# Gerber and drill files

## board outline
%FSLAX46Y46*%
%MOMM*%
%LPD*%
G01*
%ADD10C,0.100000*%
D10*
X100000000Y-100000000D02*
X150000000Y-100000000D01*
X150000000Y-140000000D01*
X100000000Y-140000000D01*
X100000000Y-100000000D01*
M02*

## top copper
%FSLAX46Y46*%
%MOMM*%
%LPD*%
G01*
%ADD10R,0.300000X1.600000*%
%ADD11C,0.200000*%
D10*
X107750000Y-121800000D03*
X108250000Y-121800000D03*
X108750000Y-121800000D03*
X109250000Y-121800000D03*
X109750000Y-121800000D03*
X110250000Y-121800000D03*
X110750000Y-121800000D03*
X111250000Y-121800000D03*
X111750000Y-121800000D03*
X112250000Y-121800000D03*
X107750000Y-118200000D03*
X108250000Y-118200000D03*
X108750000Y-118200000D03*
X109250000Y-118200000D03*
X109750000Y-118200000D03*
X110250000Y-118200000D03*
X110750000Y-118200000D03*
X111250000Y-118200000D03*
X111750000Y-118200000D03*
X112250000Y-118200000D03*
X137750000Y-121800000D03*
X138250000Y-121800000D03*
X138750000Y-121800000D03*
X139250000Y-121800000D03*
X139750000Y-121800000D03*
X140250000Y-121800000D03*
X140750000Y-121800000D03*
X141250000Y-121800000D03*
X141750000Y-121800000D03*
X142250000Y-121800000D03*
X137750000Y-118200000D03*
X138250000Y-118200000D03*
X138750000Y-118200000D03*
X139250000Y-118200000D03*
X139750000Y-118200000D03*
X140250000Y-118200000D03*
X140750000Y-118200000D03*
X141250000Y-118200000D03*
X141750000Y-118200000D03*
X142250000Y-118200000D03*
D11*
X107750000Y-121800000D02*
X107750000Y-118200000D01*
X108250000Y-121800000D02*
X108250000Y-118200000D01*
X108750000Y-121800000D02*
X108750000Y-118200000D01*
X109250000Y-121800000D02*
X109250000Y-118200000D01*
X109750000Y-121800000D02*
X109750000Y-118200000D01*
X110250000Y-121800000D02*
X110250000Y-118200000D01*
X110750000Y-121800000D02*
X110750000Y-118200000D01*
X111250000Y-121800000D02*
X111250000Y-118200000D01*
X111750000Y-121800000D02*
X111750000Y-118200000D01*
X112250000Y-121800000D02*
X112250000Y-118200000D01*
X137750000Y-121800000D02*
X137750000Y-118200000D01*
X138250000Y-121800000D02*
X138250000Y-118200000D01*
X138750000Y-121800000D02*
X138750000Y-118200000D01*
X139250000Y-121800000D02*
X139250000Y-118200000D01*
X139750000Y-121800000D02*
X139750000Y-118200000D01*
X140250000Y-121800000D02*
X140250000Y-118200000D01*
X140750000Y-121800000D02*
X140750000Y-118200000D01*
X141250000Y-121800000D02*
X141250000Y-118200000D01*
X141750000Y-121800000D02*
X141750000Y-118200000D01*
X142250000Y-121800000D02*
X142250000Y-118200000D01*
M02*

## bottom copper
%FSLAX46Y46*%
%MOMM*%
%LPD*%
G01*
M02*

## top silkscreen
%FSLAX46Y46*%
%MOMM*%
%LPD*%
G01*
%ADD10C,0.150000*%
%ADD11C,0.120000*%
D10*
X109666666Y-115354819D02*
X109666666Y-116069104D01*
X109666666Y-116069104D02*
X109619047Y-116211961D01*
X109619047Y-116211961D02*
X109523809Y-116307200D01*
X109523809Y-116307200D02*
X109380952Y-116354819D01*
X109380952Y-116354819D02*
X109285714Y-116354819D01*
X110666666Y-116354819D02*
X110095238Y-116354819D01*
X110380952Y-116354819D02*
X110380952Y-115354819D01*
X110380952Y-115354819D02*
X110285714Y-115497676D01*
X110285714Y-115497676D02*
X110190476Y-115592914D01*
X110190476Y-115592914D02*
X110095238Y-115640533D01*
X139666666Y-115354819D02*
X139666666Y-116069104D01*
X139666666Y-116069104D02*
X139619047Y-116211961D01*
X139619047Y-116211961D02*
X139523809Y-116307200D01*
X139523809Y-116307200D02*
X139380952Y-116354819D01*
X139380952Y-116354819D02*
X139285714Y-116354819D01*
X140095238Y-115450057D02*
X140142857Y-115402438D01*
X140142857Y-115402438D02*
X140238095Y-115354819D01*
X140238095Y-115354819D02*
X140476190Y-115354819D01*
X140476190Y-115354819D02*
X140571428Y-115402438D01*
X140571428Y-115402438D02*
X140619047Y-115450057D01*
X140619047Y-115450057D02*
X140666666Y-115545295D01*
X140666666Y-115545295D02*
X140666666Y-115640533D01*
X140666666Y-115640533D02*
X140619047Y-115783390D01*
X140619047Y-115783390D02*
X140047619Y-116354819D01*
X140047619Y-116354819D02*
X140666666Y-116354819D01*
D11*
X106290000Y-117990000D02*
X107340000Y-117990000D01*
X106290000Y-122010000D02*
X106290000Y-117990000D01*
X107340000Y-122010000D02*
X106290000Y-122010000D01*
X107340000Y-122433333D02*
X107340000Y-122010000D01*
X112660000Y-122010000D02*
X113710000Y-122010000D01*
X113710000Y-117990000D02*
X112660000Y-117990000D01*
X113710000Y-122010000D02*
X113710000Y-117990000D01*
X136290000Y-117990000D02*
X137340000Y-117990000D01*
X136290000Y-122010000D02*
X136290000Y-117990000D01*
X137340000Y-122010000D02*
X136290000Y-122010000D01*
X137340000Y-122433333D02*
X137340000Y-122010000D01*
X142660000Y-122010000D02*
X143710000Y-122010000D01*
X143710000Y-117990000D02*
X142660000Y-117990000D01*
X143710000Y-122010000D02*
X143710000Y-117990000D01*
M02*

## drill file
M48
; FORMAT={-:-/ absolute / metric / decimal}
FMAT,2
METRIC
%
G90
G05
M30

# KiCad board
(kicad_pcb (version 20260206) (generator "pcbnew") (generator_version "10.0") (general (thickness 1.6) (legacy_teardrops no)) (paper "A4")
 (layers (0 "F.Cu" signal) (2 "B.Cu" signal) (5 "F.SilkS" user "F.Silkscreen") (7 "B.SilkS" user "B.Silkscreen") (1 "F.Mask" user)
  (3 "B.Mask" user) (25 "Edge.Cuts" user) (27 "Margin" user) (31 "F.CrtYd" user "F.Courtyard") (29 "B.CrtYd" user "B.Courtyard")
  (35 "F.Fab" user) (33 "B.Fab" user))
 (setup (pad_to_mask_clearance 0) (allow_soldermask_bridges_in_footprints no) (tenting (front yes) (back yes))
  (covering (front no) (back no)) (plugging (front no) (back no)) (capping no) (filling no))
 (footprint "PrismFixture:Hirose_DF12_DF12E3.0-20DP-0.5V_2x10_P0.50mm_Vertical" (layer "F.Cu") (at 110 120)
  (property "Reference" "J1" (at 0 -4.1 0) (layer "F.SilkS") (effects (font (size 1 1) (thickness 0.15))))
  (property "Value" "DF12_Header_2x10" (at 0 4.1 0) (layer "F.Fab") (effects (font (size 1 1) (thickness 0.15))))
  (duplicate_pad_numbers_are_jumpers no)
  (fp_line (start -3.71 -2.01) (end -2.66 -2.01) (stroke (width 0.12) (type solid)) (layer "F.SilkS"))
  (fp_line (start -3.71 2.01) (end -3.71 -2.01) (stroke (width 0.12) (type solid)) (layer "F.SilkS"))
  (fp_line (start -2.66 2.01) (end -3.71 2.01) (stroke (width 0.12) (type solid)) (layer "F.SilkS"))
  (fp_line (start -2.66 2.433333) (end -2.66 2.01) (stroke (width 0.12) (type solid)) (layer "F.SilkS"))
  (fp_line (start 2.66 2.01) (end 3.71 2.01) (stroke (width 0.12) (type solid)) (layer "F.SilkS"))
  (fp_line (start 3.71 -2.01) (end 2.66 -2.01) (stroke (width 0.12) (type solid)) (layer "F.SilkS"))
  (fp_line (start 3.71 2.01) (end 3.71 -2.01) (stroke (width 0.12) (type solid)) (layer "F.SilkS"))
  (pad "" smd rect (at -2.25 -2) (size 0.28 1.2) (layers "F.Paste"))
  (pad "" smd rect (at -2.25 2) (size 0.28 1.2) (layers "F.Paste"))
  (pad "" smd rect (at -1.75 -2) (size 0.28 1.2) (layers "F.Paste"))
  (pad "" smd rect (at -1.75 2) (size 0.28 1.2) (layers "F.Paste"))
  (pad "" smd rect (at -1.25 -2) (size 0.28 1.2) (layers "F.Paste"))
  (pad "" smd rect (at -1.25 2) (size 0.28 1.2) (layers "F.Paste"))
  (pad "" smd rect (at -0.75 -2) (size 0.28 1.2) (layers "F.Paste"))
  (pad "" smd rect (at -0.75 2) (size 0.28 1.2) (layers "F.Paste"))
  (pad "" smd rect (at -0.25 -2) (size 0.28 1.2) (layers "F.Paste"))
  (pad "" smd rect (at -0.25 2) (size 0.28 1.2) (layers "F.Paste"))
  (pad "" smd rect (at 0.25 -2) (size 0.28 1.2) (layers "F.Paste"))
  (pad "" smd rect (at 0.25 2) (size 0.28 1.2) (layers "F.Paste"))
  (pad "" smd rect (at 0.75 -2) (size 0.28 1.2) (layers "F.Paste"))
  (pad "" smd rect (at 0.75 2) (size 0.28 1.2) (layers "F.Paste"))
  (pad "" smd rect (at 1.25 -2) (size 0.28 1.2) (layers "F.Paste"))
  (pad "" smd rect (at 1.25 2) (size 0.28 1.2) (layers "F.Paste"))
  (pad "" smd rect (at 1.75 -2) (size 0.28 1.2) (layers "F.Paste"))
  (pad "" smd rect (at 1.75 2) (size 0.28 1.2) (layers "F.Paste"))
  (pad "" smd rect (at 2.25 -2) (size 0.28 1.2) (layers "F.Paste"))
  (pad "" smd rect (at 2.25 2) (size 0.28 1.2) (layers "F.Paste"))
  (pad "1" smd rect (at -2.25 1.8) (size 0.3 1.6) (layers "F.Cu" "F.Mask") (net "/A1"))
  (pad "2" smd rect (at -1.75 1.8) (size 0.3 1.6) (layers "F.Cu" "F.Mask") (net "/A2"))
  (pad "3" smd rect (at -1.25 1.8) (size 0.3 1.6) (layers "F.Cu" "F.Mask") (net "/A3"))
  (pad "4" smd rect (at -0.75 1.8) (size 0.3 1.6) (layers "F.Cu" "F.Mask") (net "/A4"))
  (pad "5" smd rect (at -0.25 1.8) (size 0.3 1.6) (layers "F.Cu" "F.Mask") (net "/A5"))
  (pad "6" smd rect (at 0.25 1.8) (size 0.3 1.6) (layers "F.Cu" "F.Mask") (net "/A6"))
  (pad "7" smd rect (at 0.75 1.8) (size 0.3 1.6) (layers "F.Cu" "F.Mask") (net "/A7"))
  (pad "8" smd rect (at 1.25 1.8) (size 0.3 1.6) (layers "F.Cu" "F.Mask") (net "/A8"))
  (pad "9" smd rect (at 1.75 1.8) (size 0.3 1.6) (layers "F.Cu" "F.Mask") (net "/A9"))
  (pad "10" smd rect (at 2.25 1.8) (size 0.3 1.6) (layers "F.Cu" "F.Mask") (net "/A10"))
  (pad "11" smd rect (at -2.25 -1.8) (size 0.3 1.6) (layers "F.Cu" "F.Mask") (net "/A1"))
  (pad "12" smd rect (at -1.75 -1.8) (size 0.3 1.6) (layers "F.Cu" "F.Mask") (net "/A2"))
  (pad "13" smd rect (at -1.25 -1.8) (size 0.3 1.6) (layers "F.Cu" "F.Mask") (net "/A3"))
  (pad "14" smd rect (at -0.75 -1.8) (size 0.3 1.6) (layers "F.Cu" "F.Mask") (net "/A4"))
  (pad "15" smd rect (at -0.25 -1.8) (size 0.3 1.6) (layers "F.Cu" "F.Mask") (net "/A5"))
  (pad "16" smd rect (at 0.25 -1.8) (size 0.3 1.6) (layers "F.Cu" "F.Mask") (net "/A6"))
  (pad "17" smd rect (at 0.75 -1.8) (size 0.3 1.6) (layers "F.Cu" "F.Mask") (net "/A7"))
  (pad "18" smd rect (at 1.25 -1.8) (size 0.3 1.6) (layers "F.Cu" "F.Mask") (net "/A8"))
  (pad "19" smd rect (at 1.75 -1.8) (size 0.3 1.6) (layers "F.Cu" "F.Mask") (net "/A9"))
  (pad "20" smd rect (at 2.25 -1.8) (size 0.3 1.6) (layers "F.Cu" "F.Mask") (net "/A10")))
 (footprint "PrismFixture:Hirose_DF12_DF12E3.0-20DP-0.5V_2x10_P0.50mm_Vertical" (layer "F.Cu") (at 140 120)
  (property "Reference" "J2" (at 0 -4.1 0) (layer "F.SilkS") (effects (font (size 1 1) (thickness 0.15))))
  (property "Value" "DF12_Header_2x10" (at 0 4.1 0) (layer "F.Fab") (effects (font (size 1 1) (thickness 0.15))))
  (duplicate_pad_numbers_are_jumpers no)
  (fp_line (start -3.71 -2.01) (end -2.66 -2.01) (stroke (width 0.12) (type solid)) (layer "F.SilkS"))
  (fp_line (start -3.71 2.01) (end -3.71 -2.01) (stroke (width 0.12) (type solid)) (layer "F.SilkS"))
  (fp_line (start -2.66 2.01) (end -3.71 2.01) (stroke (width 0.12) (type solid)) (layer "F.SilkS"))
  (fp_line (start -2.66 2.433333) (end -2.66 2.01) (stroke (width 0.12) (type solid)) (layer "F.SilkS"))
  (fp_line (start 2.66 2.01) (end 3.71 2.01) (stroke (width 0.12) (type solid)) (layer "F.SilkS"))
  (fp_line (start 3.71 -2.01) (end 2.66 -2.01) (stroke (width 0.12) (type solid)) (layer "F.SilkS"))
  (fp_line (start 3.71 2.01) (end 3.71 -2.01) (stroke (width 0.12) (type solid)) (layer "F.SilkS"))
  (pad "" smd rect (at -2.25 -2) (size 0.28 1.2) (layers "F.Paste"))
  (pad "" smd rect (at -2.25 2) (size 0.28 1.2) (layers "F.Paste"))
  (pad "" smd rect (at -1.75 -2) (size 0.28 1.2) (layers "F.Paste"))
  (pad "" smd rect (at -1.75 2) (size 0.28 1.2) (layers "F.Paste"))
  (pad "" smd rect (at -1.25 -2) (size 0.28 1.2) (layers "F.Paste"))
  (pad "" smd rect (at -1.25 2) (size 0.28 1.2) (layers "F.Paste"))
  (pad "" smd rect (at -0.75 -2) (size 0.28 1.2) (layers "F.Paste"))
  (pad "" smd rect (at -0.75 2) (size 0.28 1.2) (layers "F.Paste"))
  (pad "" smd rect (at -0.25 -2) (size 0.28 1.2) (layers "F.Paste"))
  (pad "" smd rect (at -0.25 2) (size 0.28 1.2) (layers "F.Paste"))
  (pad "" smd rect (at 0.25 -2) (size 0.28 1.2) (layers "F.Paste"))
  (pad "" smd rect (at 0.25 2) (size 0.28 1.2) (layers "F.Paste"))
  (pad "" smd rect (at 0.75 -2) (size 0.28 1.2) (layers "F.Paste"))
  (pad "" smd rect (at 0.75 2) (size 0.28 1.2) (layers "F.Paste"))
  (pad "" smd rect (at 1.25 -2) (size 0.28 1.2) (layers "F.Paste"))
  (pad "" smd rect (at 1.25 2) (size 0.28 1.2) (layers "F.Paste"))
  (pad "" smd rect (at 1.75 -2) (size 0.28 1.2) (layers "F.Paste"))
  (pad "" smd rect (at 1.75 2) (size 0.28 1.2) (layers "F.Paste"))
  (pad "" smd rect (at 2.25 -2) (size 0.28 1.2) (layers "F.Paste"))
  (pad "" smd rect (at 2.25 2) (size 0.28 1.2) (layers "F.Paste"))
  (pad "1" smd rect (at -2.25 1.8) (size 0.3 1.6) (layers "F.Cu" "F.Mask") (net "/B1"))
  (pad "2" smd rect (at -1.75 1.8) (size 0.3 1.6) (layers "F.Cu" "F.Mask") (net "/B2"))
  (pad "3" smd rect (at -1.25 1.8) (size 0.3 1.6) (layers "F.Cu" "F.Mask") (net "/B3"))
  (pad "4" smd rect (at -0.75 1.8) (size 0.3 1.6) (layers "F.Cu" "F.Mask") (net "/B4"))
  (pad "5" smd rect (at -0.25 1.8) (size 0.3 1.6) (layers "F.Cu" "F.Mask") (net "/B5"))
  (pad "6" smd rect (at 0.25 1.8) (size 0.3 1.6) (layers "F.Cu" "F.Mask") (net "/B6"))
  (pad "7" smd rect (at 0.75 1.8) (size 0.3 1.6) (layers "F.Cu" "F.Mask") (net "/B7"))
  (pad "8" smd rect (at 1.25 1.8) (size 0.3 1.6) (layers "F.Cu" "F.Mask") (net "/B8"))
  (pad "9" smd rect (at 1.75 1.8) (size 0.3 1.6) (layers "F.Cu" "F.Mask") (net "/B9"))
  (pad "10" smd rect (at 2.25 1.8) (size 0.3 1.6) (layers "F.Cu" "F.Mask") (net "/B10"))
  (pad "11" smd rect (at -2.25 -1.8) (size 0.3 1.6) (layers "F.Cu" "F.Mask") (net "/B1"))
  (pad "12" smd rect (at -1.75 -1.8) (size 0.3 1.6) (layers "F.Cu" "F.Mask") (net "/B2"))
  (pad "13" smd rect (at -1.25 -1.8) (size 0.3 1.6) (layers "F.Cu" "F.Mask") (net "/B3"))
  (pad "14" smd rect (at -0.75 -1.8) (size 0.3 1.6) (layers "F.Cu" "F.Mask") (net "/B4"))
  (pad "15" smd rect (at -0.25 -1.8) (size 0.3 1.6) (layers "F.Cu" "F.Mask") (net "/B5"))
  (pad "16" smd rect (at 0.25 -1.8) (size 0.3 1.6) (layers "F.Cu" "F.Mask") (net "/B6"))
  (pad "17" smd rect (at 0.75 -1.8) (size 0.3 1.6) (layers "F.Cu" "F.Mask") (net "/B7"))
  (pad "18" smd rect (at 1.25 -1.8) (size 0.3 1.6) (layers "F.Cu" "F.Mask") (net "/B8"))
  (pad "19" smd rect (at 1.75 -1.8) (size 0.3 1.6) (layers "F.Cu" "F.Mask") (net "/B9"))
  (pad "20" smd rect (at 2.25 -1.8) (size 0.3 1.6) (layers "F.Cu" "F.Mask") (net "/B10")))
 (gr_rect (start 100 100) (end 150 140) (stroke (width 0.1) (type solid)) (fill no) (layer "Edge.Cuts"))
 (segment (start 107.75 121.8) (end 107.75 118.2) (width 0.2) (layer "F.Cu") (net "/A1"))
 (segment (start 108.25 121.8) (end 108.25 118.2) (width 0.2) (layer "F.Cu") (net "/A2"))
 (segment (start 108.75 121.8) (end 108.75 118.2) (width 0.2) (layer "F.Cu") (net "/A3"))
 (segment (start 109.25 121.8) (end 109.25 118.2) (width 0.2) (layer "F.Cu") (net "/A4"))
 (segment (start 109.75 121.8) (end 109.75 118.2) (width 0.2) (layer "F.Cu") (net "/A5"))
 (segment (start 110.25 121.8) (end 110.25 118.2) (width 0.2) (layer "F.Cu") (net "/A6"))
 (segment (start 110.75 121.8) (end 110.75 118.2) (width 0.2) (layer "F.Cu") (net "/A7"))
 (segment (start 111.25 121.8) (end 111.25 118.2) (width 0.2) (layer "F.Cu") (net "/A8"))
 (segment (start 111.75 121.8) (end 111.75 118.2) (width 0.2) (layer "F.Cu") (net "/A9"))
 (segment (start 112.25 121.8) (end 112.25 118.2) (width 0.2) (layer "F.Cu") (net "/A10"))
 (segment (start 137.75 121.8) (end 137.75 118.2) (width 0.2) (layer "F.Cu") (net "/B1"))
 (segment (start 138.25 121.8) (end 138.25 118.2) (width 0.2) (layer "F.Cu") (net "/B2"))
 (segment (start 138.75 121.8) (end 138.75 118.2) (width 0.2) (layer "F.Cu") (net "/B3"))
 (segment (start 139.25 121.8) (end 139.25 118.2) (width 0.2) (layer "F.Cu") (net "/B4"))
 (segment (start 139.75 121.8) (end 139.75 118.2) (width 0.2) (layer "F.Cu") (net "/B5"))
 (segment (start 140.25 121.8) (end 140.25 118.2) (width 0.2) (layer "F.Cu") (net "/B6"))
 (segment (start 140.75 121.8) (end 140.75 118.2) (width 0.2) (layer "F.Cu") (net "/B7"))
 (segment (start 141.25 121.8) (end 141.25 118.2) (width 0.2) (layer "F.Cu") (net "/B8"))
 (segment (start 141.75 121.8) (end 141.75 118.2) (width 0.2) (layer "F.Cu") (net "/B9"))
 (segment (start 142.25 121.8) (end 142.25 118.2) (width 0.2) (layer "F.Cu") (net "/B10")))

